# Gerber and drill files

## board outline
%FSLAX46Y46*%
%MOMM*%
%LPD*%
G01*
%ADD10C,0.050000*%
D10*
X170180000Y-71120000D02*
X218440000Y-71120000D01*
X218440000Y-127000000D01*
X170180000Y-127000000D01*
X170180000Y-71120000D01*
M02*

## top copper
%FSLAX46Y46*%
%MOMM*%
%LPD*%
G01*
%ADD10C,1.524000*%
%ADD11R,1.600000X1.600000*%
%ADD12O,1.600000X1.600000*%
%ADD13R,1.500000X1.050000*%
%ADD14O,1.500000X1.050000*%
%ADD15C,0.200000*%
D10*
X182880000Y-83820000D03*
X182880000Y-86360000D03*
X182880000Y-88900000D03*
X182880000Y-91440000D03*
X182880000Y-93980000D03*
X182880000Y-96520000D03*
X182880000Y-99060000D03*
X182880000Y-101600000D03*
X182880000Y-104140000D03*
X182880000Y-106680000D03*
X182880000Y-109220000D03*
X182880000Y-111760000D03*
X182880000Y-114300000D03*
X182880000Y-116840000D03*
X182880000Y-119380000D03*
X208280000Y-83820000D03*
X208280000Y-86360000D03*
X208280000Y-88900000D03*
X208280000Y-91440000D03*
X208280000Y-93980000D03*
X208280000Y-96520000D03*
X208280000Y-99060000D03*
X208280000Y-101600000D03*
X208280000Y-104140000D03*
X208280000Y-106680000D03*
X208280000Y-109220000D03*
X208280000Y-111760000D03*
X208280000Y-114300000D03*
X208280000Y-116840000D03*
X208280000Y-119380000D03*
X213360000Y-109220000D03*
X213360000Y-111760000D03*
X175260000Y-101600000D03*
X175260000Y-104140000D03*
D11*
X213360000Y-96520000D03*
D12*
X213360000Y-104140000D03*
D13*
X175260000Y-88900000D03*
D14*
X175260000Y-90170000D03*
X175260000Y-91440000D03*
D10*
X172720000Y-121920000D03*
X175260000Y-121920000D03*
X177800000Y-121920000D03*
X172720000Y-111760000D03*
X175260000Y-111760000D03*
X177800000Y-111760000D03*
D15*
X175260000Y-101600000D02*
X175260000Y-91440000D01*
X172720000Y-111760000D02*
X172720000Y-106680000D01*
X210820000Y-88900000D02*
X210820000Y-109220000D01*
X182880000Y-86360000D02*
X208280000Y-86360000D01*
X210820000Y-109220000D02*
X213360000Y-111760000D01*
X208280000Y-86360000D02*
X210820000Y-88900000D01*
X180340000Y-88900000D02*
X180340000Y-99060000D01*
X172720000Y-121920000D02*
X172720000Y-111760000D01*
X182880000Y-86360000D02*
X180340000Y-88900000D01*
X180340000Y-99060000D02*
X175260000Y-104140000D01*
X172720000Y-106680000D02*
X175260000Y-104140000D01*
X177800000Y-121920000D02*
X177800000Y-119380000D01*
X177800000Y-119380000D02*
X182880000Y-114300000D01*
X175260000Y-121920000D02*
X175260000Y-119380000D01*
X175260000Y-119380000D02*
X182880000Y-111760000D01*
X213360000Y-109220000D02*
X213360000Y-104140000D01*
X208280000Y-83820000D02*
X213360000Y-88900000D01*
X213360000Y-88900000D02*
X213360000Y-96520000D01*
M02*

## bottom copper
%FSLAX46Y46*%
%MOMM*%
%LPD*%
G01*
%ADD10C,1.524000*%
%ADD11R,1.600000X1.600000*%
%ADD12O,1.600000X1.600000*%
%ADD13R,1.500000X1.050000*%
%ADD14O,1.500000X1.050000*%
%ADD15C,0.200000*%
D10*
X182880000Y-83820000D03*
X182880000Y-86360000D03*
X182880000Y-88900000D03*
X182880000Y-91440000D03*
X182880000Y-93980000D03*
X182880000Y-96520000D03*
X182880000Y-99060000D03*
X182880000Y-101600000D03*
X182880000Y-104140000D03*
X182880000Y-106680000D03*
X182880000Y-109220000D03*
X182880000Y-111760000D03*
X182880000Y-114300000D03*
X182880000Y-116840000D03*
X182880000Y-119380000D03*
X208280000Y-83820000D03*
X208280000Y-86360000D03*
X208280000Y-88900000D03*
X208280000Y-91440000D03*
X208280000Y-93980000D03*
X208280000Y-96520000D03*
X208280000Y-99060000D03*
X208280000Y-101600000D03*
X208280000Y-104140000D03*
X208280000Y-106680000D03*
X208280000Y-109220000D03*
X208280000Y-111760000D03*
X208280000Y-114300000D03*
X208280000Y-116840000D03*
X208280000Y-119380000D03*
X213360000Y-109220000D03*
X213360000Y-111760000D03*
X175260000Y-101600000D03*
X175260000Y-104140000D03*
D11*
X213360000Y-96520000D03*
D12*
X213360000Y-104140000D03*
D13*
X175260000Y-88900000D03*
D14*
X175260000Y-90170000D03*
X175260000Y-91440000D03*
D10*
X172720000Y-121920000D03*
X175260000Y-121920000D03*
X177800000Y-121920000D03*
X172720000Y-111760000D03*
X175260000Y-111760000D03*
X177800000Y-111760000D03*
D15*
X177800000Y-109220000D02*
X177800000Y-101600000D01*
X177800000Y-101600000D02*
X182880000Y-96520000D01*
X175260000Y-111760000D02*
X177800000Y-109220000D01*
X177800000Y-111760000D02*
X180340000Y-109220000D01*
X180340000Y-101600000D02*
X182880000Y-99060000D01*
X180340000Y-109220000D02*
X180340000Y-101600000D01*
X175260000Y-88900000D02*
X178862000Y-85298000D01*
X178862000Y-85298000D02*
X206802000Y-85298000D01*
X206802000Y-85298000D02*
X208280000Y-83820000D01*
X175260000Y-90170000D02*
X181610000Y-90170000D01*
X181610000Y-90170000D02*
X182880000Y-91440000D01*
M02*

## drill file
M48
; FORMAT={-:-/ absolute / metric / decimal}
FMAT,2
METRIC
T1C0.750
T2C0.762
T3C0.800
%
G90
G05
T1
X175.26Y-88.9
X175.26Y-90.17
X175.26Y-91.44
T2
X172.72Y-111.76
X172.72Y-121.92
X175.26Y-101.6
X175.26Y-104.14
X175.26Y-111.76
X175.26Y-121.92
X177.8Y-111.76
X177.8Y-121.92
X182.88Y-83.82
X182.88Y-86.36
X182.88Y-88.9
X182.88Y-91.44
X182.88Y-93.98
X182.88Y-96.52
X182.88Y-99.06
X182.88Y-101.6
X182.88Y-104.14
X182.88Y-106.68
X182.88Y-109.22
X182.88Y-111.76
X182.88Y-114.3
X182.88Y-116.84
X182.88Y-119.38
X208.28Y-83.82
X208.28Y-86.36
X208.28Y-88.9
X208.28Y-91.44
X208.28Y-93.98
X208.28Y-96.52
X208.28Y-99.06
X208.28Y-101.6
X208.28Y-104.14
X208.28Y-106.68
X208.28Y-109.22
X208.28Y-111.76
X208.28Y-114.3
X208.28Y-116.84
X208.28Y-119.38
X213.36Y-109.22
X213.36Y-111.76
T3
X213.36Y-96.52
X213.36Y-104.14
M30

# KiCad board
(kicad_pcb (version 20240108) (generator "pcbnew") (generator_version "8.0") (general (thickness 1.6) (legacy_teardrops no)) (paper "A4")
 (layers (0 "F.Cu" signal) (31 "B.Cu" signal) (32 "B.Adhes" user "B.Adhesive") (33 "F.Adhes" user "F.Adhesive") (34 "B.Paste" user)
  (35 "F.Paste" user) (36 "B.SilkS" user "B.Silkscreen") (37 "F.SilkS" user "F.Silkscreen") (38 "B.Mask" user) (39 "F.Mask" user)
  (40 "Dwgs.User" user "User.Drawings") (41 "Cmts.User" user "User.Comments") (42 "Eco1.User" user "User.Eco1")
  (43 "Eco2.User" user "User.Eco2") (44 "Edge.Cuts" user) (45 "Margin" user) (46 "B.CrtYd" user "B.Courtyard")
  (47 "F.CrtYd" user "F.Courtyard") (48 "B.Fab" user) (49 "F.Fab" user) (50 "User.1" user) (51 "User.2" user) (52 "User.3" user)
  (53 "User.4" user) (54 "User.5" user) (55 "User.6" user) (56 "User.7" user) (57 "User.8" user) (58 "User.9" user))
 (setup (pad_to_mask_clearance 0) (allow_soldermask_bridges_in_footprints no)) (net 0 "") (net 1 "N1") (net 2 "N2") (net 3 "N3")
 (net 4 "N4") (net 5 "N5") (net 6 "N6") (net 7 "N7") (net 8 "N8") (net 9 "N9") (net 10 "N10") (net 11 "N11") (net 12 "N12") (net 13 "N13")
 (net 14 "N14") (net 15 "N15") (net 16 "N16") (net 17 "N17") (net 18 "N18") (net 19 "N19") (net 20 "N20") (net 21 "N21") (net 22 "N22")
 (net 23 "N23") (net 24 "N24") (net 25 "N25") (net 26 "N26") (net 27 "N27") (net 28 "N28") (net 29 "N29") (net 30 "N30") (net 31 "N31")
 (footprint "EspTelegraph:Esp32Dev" (layer "F.Cu") (at 195.58 83.82)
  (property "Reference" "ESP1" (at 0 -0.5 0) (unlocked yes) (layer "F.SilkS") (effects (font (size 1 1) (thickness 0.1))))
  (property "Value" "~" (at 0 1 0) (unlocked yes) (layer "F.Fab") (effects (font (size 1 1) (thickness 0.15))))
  (pad "1" thru_hole circle (at -12.7 0) (size 1.524 1.524) (drill 0.762) (layers "*.Cu" "*.Mask") (remove_unused_layers no) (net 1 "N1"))
  (pad "2" thru_hole circle (at -12.7 2.54) (size 1.524 1.524) (drill 0.762) (layers "*.Cu" "*.Mask") (remove_unused_layers no) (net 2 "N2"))
  (pad "3" thru_hole circle (at -12.7 5.08) (size 1.524 1.524) (drill 0.762) (layers "*.Cu" "*.Mask") (remove_unused_layers no) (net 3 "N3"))
  (pad "4" thru_hole circle (at -12.7 7.62) (size 1.524 1.524) (drill 0.762) (layers "*.Cu" "*.Mask") (remove_unused_layers no) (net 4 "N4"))
  (pad "5" thru_hole circle (at -12.7 10.16) (size 1.524 1.524) (drill 0.762) (layers "*.Cu" "*.Mask") (remove_unused_layers no)
   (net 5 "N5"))
  (pad "6" thru_hole circle (at -12.7 12.7) (size 1.524 1.524) (drill 0.762) (layers "*.Cu" "*.Mask") (remove_unused_layers no) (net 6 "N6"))
  (pad "7" thru_hole circle (at -12.7 15.24) (size 1.524 1.524) (drill 0.762) (layers "*.Cu" "*.Mask") (remove_unused_layers no)
   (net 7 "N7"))
  (pad "8" thru_hole circle (at -12.7 17.78) (size 1.524 1.524) (drill 0.762) (layers "*.Cu" "*.Mask") (remove_unused_layers no)
   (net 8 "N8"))
  (pad "9" thru_hole circle (at -12.7 20.32) (size 1.524 1.524) (drill 0.762) (layers "*.Cu" "*.Mask") (remove_unused_layers no)
   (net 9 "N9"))
  (pad "10" thru_hole circle (at -12.7 22.86) (size 1.524 1.524) (drill 0.762) (layers "*.Cu" "*.Mask") (remove_unused_layers no)
   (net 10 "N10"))
  (pad "11" thru_hole circle (at -12.7 25.4) (size 1.524 1.524) (drill 0.762) (layers "*.Cu" "*.Mask") (remove_unused_layers no)
   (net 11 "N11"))
  (pad "12" thru_hole circle (at -12.7 27.94) (size 1.524 1.524) (drill 0.762) (layers "*.Cu" "*.Mask") (remove_unused_layers no)
   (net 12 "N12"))
  (pad "13" thru_hole circle (at -12.7 30.48) (size 1.524 1.524) (drill 0.762) (layers "*.Cu" "*.Mask") (remove_unused_layers no)
   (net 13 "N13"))
  (pad "14" thru_hole circle (at -12.7 33.02) (size 1.524 1.524) (drill 0.762) (layers "*.Cu" "*.Mask") (remove_unused_layers no)
   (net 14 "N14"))
  (pad "15" thru_hole circle (at -12.7 35.56) (size 1.524 1.524) (drill 0.762) (layers "*.Cu" "*.Mask") (remove_unused_layers no)
   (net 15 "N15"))
  (pad "16" thru_hole circle (at 12.7 0) (size 1.524 1.524) (drill 0.762) (layers "*.Cu" "*.Mask") (remove_unused_layers no) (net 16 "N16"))
  (pad "17" thru_hole circle (at 12.7 2.54) (size 1.524 1.524) (drill 0.762) (layers "*.Cu" "*.Mask") (remove_unused_layers no) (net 2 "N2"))
  (pad "18" thru_hole circle (at 12.7 5.08) (size 1.524 1.524) (drill 0.762) (layers "*.Cu" "*.Mask") (remove_unused_layers no)
   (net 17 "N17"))
  (pad "19" thru_hole circle (at 12.7 7.62) (size 1.524 1.524) (drill 0.762) (layers "*.Cu" "*.Mask") (remove_unused_layers no)
   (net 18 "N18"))
  (pad "20" thru_hole circle (at 12.7 10.16) (size 1.524 1.524) (drill 0.762) (layers "*.Cu" "*.Mask") (remove_unused_layers no)
   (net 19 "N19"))
  (pad "21" thru_hole circle (at 12.7 12.7) (size 1.524 1.524) (drill 0.762) (layers "*.Cu" "*.Mask") (remove_unused_layers no)
   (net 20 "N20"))
  (pad "22" thru_hole circle (at 12.7 15.24) (size 1.524 1.524) (drill 0.762) (layers "*.Cu" "*.Mask") (remove_unused_layers no)
   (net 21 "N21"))
  (pad "23" thru_hole circle (at 12.7 17.78) (size 1.524 1.524) (drill 0.762) (layers "*.Cu" "*.Mask") (remove_unused_layers no)
   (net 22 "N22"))
  (pad "24" thru_hole circle (at 12.7 20.32) (size 1.524 1.524) (drill 0.762) (layers "*.Cu" "*.Mask") (remove_unused_layers no)
   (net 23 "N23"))
  (pad "25" thru_hole circle (at 12.7 22.86) (size 1.524 1.524) (drill 0.762) (layers "*.Cu" "*.Mask") (remove_unused_layers no)
   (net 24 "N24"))
  (pad "26" thru_hole circle (at 12.7 25.4) (size 1.524 1.524) (drill 0.762) (layers "*.Cu" "*.Mask") (remove_unused_layers no)
   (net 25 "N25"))
  (pad "27" thru_hole circle (at 12.7 27.94) (size 1.524 1.524) (drill 0.762) (layers "*.Cu" "*.Mask") (remove_unused_layers no)
   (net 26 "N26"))
  (pad "28" thru_hole circle (at 12.7 30.48) (size 1.524 1.524) (drill 0.762) (layers "*.Cu" "*.Mask") (remove_unused_layers no)
   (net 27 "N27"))
  (pad "29" thru_hole circle (at 12.7 33.02) (size 1.524 1.524) (drill 0.762) (layers "*.Cu" "*.Mask") (remove_unused_layers no)
   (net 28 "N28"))
  (pad "30" thru_hole circle (at 12.7 35.56) (size 1.524 1.524) (drill 0.762) (layers "*.Cu" "*.Mask") (remove_unused_layers no)
   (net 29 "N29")))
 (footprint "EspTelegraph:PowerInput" (layer "F.Cu") (at 213.36 109.22 -90)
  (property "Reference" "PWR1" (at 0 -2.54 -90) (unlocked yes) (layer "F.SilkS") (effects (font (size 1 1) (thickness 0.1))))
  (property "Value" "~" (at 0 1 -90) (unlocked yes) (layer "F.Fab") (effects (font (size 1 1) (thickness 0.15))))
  (pad "1" thru_hole circle (at 0 0 270) (size 1.524 1.524) (drill 0.762) (layers "*.Cu" "*.Mask") (remove_unused_layers no) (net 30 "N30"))
  (pad "2" thru_hole circle (at 2.54 0 270) (size 1.524 1.524) (drill 0.762) (layers "*.Cu" "*.Mask") (remove_unused_layers no) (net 2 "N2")))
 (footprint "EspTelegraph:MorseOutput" (layer "F.Cu") (at 175.26 101.6 -90)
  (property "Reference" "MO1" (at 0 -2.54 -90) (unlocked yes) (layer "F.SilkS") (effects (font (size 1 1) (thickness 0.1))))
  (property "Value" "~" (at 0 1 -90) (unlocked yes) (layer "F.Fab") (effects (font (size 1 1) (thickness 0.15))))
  (pad "1" thru_hole circle (at 0 0 270) (size 1.524 1.524) (drill 0.762) (layers "*.Cu" "*.Mask") (remove_unused_layers no) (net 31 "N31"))
  (pad "2" thru_hole circle (at 2.54 0 270) (size 1.524 1.524) (drill 0.762) (layers "*.Cu" "*.Mask") (remove_unused_layers no) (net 2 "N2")))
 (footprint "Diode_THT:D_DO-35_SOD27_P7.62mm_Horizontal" (layer "F.Cu") (at 213.36 96.52 -90)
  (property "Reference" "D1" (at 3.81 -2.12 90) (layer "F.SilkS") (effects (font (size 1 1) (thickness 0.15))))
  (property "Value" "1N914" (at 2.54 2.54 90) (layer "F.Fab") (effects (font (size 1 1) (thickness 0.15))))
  (pad "1" thru_hole rect (at 0 0 270) (size 1.6 1.6) (drill 0.8) (layers "*.Cu" "*.Mask") (remove_unused_layers no) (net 16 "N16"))
  (pad "2" thru_hole oval (at 7.62 0 270) (size 1.6 1.6) (drill 0.8) (layers "*.Cu" "*.Mask") (remove_unused_layers no) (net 30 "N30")))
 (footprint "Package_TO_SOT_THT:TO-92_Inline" (layer "F.Cu") (at 175.26 88.9 -90)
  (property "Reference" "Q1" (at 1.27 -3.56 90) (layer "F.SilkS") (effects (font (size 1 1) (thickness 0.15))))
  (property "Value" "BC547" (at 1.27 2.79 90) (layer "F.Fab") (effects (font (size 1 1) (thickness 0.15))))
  (pad "1" thru_hole rect (at 0 0 270) (size 1.05 1.5) (drill 0.75) (layers "*.Cu" "*.Mask") (remove_unused_layers no) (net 16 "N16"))
  (pad "2" thru_hole oval (at 1.27 0 270) (size 1.05 1.5) (drill 0.75) (layers "*.Cu" "*.Mask") (remove_unused_layers no) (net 4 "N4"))
  (pad "3" thru_hole oval (at 2.54 0 270) (size 1.05 1.5) (drill 0.75) (layers "*.Cu" "*.Mask") (remove_unused_layers no) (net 31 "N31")))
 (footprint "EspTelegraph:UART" (layer "F.Cu") (at 172.72 121.92)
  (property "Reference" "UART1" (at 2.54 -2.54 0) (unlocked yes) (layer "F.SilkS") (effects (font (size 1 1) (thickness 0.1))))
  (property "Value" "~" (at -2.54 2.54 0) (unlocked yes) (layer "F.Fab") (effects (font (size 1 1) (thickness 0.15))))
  (pad "1" thru_hole circle (at 0 0) (size 1.524 1.524) (drill 0.762) (layers "*.Cu" "*.Mask") (remove_unused_layers no) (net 2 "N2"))
  (pad "2" thru_hole circle (at 2.54 0) (size 1.524 1.524) (drill 0.762) (layers "*.Cu" "*.Mask") (remove_unused_layers no) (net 12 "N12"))
  (pad "3" thru_hole circle (at 5.08 0) (size 1.524 1.524) (drill 0.762) (layers "*.Cu" "*.Mask") (remove_unused_layers no) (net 13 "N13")))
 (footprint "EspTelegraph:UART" (layer "F.Cu") (at 172.72 111.76)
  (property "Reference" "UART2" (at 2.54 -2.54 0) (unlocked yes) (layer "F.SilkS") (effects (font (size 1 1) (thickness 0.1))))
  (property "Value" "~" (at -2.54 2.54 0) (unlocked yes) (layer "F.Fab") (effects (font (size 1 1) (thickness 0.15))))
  (pad "1" thru_hole circle (at 0 0) (size 1.524 1.524) (drill 0.762) (layers "*.Cu" "*.Mask") (remove_unused_layers no) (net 2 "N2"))
  (pad "2" thru_hole circle (at 2.54 0) (size 1.524 1.524) (drill 0.762) (layers "*.Cu" "*.Mask") (remove_unused_layers no) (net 6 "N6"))
  (pad "3" thru_hole circle (at 5.08 0) (size 1.524 1.524) (drill 0.762) (layers "*.Cu" "*.Mask") (remove_unused_layers no) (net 7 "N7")))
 (gr_rect (start 170.18 71.12) (end 218.44 127) (stroke (width 0.05) (type default)) (fill none) (layer "Edge.Cuts"))
 (segment (start 175.26 101.6) (end 175.26 91.44) (width 0.2) (layer "F.Cu") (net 31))
 (segment (start 172.72 111.76) (end 172.72 106.68) (width 0.2) (layer "F.Cu") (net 2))
 (segment (start 210.82 88.9) (end 210.82 109.22) (width 0.2) (layer "F.Cu") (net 2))
 (segment (start 182.88 86.36) (end 208.28 86.36) (width 0.2) (layer "F.Cu") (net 2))
 (segment (start 210.82 109.22) (end 213.36 111.76) (width 0.2) (layer "F.Cu") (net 2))
 (segment (start 208.28 86.36) (end 210.82 88.9) (width 0.2) (layer "F.Cu") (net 2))
 (segment (start 180.34 88.9) (end 180.34 99.06) (width 0.2) (layer "F.Cu") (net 2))
 (segment (start 172.72 121.92) (end 172.72 111.76) (width 0.2) (layer "F.Cu") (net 2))
 (segment (start 182.88 86.36) (end 180.34 88.9) (width 0.2) (layer "F.Cu") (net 2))
 (segment (start 180.34 99.06) (end 175.26 104.14) (width 0.2) (layer "F.Cu") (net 2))
 (segment (start 172.72 106.68) (end 175.26 104.14) (width 0.2) (layer "F.Cu") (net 2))
 (segment (start 177.8 121.92) (end 177.8 119.38) (width 0.2) (layer "F.Cu") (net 13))
 (segment (start 177.8 119.38) (end 182.88 114.3) (width 0.2) (layer "F.Cu") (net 13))
 (segment (start 177.8 109.22) (end 177.8 101.6) (width 0.2) (layer "B.Cu") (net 6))
 (segment (start 177.8 101.6) (end 182.88 96.52) (width 0.2) (layer "B.Cu") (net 6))
 (segment (start 175.26 111.76) (end 177.8 109.22) (width 0.2) (layer "B.Cu") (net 6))
 (segment (start 177.8 111.76) (end 180.34 109.22) (width 0.2) (layer "B.Cu") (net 7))
 (segment (start 180.34 101.6) (end 182.88 99.06) (width 0.2) (layer "B.Cu") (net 7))
 (segment (start 180.34 109.22) (end 180.34 101.6) (width 0.2) (layer "B.Cu") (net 7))
 (segment (start 175.26 121.92) (end 175.26 119.38) (width 0.2) (layer "F.Cu") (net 12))
 (segment (start 175.26 119.38) (end 182.88 111.76) (width 0.2) (layer "F.Cu") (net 12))
 (segment (start 213.36 109.22) (end 213.36 104.14) (width 0.2) (layer "F.Cu") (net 30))
 (segment (start 208.28 83.82) (end 213.36 88.9) (width 0.2) (layer "F.Cu") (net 16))
 (segment (start 213.36 88.9) (end 213.36 96.52) (width 0.2) (layer "F.Cu") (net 16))
 (segment (start 175.26 88.9) (end 178.862 85.298) (width 0.2) (layer "B.Cu") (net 16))
 (segment (start 178.862 85.298) (end 206.802 85.298) (width 0.2) (layer "B.Cu") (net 16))
 (segment (start 206.802 85.298) (end 208.28 83.82) (width 0.2) (layer "B.Cu") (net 16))
 (segment (start 175.26 90.17) (end 181.61 90.17) (width 0.2) (layer "B.Cu") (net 4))
 (segment (start 181.61 90.17) (end 182.88 91.44) (width 0.2) (layer "B.Cu") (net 4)))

